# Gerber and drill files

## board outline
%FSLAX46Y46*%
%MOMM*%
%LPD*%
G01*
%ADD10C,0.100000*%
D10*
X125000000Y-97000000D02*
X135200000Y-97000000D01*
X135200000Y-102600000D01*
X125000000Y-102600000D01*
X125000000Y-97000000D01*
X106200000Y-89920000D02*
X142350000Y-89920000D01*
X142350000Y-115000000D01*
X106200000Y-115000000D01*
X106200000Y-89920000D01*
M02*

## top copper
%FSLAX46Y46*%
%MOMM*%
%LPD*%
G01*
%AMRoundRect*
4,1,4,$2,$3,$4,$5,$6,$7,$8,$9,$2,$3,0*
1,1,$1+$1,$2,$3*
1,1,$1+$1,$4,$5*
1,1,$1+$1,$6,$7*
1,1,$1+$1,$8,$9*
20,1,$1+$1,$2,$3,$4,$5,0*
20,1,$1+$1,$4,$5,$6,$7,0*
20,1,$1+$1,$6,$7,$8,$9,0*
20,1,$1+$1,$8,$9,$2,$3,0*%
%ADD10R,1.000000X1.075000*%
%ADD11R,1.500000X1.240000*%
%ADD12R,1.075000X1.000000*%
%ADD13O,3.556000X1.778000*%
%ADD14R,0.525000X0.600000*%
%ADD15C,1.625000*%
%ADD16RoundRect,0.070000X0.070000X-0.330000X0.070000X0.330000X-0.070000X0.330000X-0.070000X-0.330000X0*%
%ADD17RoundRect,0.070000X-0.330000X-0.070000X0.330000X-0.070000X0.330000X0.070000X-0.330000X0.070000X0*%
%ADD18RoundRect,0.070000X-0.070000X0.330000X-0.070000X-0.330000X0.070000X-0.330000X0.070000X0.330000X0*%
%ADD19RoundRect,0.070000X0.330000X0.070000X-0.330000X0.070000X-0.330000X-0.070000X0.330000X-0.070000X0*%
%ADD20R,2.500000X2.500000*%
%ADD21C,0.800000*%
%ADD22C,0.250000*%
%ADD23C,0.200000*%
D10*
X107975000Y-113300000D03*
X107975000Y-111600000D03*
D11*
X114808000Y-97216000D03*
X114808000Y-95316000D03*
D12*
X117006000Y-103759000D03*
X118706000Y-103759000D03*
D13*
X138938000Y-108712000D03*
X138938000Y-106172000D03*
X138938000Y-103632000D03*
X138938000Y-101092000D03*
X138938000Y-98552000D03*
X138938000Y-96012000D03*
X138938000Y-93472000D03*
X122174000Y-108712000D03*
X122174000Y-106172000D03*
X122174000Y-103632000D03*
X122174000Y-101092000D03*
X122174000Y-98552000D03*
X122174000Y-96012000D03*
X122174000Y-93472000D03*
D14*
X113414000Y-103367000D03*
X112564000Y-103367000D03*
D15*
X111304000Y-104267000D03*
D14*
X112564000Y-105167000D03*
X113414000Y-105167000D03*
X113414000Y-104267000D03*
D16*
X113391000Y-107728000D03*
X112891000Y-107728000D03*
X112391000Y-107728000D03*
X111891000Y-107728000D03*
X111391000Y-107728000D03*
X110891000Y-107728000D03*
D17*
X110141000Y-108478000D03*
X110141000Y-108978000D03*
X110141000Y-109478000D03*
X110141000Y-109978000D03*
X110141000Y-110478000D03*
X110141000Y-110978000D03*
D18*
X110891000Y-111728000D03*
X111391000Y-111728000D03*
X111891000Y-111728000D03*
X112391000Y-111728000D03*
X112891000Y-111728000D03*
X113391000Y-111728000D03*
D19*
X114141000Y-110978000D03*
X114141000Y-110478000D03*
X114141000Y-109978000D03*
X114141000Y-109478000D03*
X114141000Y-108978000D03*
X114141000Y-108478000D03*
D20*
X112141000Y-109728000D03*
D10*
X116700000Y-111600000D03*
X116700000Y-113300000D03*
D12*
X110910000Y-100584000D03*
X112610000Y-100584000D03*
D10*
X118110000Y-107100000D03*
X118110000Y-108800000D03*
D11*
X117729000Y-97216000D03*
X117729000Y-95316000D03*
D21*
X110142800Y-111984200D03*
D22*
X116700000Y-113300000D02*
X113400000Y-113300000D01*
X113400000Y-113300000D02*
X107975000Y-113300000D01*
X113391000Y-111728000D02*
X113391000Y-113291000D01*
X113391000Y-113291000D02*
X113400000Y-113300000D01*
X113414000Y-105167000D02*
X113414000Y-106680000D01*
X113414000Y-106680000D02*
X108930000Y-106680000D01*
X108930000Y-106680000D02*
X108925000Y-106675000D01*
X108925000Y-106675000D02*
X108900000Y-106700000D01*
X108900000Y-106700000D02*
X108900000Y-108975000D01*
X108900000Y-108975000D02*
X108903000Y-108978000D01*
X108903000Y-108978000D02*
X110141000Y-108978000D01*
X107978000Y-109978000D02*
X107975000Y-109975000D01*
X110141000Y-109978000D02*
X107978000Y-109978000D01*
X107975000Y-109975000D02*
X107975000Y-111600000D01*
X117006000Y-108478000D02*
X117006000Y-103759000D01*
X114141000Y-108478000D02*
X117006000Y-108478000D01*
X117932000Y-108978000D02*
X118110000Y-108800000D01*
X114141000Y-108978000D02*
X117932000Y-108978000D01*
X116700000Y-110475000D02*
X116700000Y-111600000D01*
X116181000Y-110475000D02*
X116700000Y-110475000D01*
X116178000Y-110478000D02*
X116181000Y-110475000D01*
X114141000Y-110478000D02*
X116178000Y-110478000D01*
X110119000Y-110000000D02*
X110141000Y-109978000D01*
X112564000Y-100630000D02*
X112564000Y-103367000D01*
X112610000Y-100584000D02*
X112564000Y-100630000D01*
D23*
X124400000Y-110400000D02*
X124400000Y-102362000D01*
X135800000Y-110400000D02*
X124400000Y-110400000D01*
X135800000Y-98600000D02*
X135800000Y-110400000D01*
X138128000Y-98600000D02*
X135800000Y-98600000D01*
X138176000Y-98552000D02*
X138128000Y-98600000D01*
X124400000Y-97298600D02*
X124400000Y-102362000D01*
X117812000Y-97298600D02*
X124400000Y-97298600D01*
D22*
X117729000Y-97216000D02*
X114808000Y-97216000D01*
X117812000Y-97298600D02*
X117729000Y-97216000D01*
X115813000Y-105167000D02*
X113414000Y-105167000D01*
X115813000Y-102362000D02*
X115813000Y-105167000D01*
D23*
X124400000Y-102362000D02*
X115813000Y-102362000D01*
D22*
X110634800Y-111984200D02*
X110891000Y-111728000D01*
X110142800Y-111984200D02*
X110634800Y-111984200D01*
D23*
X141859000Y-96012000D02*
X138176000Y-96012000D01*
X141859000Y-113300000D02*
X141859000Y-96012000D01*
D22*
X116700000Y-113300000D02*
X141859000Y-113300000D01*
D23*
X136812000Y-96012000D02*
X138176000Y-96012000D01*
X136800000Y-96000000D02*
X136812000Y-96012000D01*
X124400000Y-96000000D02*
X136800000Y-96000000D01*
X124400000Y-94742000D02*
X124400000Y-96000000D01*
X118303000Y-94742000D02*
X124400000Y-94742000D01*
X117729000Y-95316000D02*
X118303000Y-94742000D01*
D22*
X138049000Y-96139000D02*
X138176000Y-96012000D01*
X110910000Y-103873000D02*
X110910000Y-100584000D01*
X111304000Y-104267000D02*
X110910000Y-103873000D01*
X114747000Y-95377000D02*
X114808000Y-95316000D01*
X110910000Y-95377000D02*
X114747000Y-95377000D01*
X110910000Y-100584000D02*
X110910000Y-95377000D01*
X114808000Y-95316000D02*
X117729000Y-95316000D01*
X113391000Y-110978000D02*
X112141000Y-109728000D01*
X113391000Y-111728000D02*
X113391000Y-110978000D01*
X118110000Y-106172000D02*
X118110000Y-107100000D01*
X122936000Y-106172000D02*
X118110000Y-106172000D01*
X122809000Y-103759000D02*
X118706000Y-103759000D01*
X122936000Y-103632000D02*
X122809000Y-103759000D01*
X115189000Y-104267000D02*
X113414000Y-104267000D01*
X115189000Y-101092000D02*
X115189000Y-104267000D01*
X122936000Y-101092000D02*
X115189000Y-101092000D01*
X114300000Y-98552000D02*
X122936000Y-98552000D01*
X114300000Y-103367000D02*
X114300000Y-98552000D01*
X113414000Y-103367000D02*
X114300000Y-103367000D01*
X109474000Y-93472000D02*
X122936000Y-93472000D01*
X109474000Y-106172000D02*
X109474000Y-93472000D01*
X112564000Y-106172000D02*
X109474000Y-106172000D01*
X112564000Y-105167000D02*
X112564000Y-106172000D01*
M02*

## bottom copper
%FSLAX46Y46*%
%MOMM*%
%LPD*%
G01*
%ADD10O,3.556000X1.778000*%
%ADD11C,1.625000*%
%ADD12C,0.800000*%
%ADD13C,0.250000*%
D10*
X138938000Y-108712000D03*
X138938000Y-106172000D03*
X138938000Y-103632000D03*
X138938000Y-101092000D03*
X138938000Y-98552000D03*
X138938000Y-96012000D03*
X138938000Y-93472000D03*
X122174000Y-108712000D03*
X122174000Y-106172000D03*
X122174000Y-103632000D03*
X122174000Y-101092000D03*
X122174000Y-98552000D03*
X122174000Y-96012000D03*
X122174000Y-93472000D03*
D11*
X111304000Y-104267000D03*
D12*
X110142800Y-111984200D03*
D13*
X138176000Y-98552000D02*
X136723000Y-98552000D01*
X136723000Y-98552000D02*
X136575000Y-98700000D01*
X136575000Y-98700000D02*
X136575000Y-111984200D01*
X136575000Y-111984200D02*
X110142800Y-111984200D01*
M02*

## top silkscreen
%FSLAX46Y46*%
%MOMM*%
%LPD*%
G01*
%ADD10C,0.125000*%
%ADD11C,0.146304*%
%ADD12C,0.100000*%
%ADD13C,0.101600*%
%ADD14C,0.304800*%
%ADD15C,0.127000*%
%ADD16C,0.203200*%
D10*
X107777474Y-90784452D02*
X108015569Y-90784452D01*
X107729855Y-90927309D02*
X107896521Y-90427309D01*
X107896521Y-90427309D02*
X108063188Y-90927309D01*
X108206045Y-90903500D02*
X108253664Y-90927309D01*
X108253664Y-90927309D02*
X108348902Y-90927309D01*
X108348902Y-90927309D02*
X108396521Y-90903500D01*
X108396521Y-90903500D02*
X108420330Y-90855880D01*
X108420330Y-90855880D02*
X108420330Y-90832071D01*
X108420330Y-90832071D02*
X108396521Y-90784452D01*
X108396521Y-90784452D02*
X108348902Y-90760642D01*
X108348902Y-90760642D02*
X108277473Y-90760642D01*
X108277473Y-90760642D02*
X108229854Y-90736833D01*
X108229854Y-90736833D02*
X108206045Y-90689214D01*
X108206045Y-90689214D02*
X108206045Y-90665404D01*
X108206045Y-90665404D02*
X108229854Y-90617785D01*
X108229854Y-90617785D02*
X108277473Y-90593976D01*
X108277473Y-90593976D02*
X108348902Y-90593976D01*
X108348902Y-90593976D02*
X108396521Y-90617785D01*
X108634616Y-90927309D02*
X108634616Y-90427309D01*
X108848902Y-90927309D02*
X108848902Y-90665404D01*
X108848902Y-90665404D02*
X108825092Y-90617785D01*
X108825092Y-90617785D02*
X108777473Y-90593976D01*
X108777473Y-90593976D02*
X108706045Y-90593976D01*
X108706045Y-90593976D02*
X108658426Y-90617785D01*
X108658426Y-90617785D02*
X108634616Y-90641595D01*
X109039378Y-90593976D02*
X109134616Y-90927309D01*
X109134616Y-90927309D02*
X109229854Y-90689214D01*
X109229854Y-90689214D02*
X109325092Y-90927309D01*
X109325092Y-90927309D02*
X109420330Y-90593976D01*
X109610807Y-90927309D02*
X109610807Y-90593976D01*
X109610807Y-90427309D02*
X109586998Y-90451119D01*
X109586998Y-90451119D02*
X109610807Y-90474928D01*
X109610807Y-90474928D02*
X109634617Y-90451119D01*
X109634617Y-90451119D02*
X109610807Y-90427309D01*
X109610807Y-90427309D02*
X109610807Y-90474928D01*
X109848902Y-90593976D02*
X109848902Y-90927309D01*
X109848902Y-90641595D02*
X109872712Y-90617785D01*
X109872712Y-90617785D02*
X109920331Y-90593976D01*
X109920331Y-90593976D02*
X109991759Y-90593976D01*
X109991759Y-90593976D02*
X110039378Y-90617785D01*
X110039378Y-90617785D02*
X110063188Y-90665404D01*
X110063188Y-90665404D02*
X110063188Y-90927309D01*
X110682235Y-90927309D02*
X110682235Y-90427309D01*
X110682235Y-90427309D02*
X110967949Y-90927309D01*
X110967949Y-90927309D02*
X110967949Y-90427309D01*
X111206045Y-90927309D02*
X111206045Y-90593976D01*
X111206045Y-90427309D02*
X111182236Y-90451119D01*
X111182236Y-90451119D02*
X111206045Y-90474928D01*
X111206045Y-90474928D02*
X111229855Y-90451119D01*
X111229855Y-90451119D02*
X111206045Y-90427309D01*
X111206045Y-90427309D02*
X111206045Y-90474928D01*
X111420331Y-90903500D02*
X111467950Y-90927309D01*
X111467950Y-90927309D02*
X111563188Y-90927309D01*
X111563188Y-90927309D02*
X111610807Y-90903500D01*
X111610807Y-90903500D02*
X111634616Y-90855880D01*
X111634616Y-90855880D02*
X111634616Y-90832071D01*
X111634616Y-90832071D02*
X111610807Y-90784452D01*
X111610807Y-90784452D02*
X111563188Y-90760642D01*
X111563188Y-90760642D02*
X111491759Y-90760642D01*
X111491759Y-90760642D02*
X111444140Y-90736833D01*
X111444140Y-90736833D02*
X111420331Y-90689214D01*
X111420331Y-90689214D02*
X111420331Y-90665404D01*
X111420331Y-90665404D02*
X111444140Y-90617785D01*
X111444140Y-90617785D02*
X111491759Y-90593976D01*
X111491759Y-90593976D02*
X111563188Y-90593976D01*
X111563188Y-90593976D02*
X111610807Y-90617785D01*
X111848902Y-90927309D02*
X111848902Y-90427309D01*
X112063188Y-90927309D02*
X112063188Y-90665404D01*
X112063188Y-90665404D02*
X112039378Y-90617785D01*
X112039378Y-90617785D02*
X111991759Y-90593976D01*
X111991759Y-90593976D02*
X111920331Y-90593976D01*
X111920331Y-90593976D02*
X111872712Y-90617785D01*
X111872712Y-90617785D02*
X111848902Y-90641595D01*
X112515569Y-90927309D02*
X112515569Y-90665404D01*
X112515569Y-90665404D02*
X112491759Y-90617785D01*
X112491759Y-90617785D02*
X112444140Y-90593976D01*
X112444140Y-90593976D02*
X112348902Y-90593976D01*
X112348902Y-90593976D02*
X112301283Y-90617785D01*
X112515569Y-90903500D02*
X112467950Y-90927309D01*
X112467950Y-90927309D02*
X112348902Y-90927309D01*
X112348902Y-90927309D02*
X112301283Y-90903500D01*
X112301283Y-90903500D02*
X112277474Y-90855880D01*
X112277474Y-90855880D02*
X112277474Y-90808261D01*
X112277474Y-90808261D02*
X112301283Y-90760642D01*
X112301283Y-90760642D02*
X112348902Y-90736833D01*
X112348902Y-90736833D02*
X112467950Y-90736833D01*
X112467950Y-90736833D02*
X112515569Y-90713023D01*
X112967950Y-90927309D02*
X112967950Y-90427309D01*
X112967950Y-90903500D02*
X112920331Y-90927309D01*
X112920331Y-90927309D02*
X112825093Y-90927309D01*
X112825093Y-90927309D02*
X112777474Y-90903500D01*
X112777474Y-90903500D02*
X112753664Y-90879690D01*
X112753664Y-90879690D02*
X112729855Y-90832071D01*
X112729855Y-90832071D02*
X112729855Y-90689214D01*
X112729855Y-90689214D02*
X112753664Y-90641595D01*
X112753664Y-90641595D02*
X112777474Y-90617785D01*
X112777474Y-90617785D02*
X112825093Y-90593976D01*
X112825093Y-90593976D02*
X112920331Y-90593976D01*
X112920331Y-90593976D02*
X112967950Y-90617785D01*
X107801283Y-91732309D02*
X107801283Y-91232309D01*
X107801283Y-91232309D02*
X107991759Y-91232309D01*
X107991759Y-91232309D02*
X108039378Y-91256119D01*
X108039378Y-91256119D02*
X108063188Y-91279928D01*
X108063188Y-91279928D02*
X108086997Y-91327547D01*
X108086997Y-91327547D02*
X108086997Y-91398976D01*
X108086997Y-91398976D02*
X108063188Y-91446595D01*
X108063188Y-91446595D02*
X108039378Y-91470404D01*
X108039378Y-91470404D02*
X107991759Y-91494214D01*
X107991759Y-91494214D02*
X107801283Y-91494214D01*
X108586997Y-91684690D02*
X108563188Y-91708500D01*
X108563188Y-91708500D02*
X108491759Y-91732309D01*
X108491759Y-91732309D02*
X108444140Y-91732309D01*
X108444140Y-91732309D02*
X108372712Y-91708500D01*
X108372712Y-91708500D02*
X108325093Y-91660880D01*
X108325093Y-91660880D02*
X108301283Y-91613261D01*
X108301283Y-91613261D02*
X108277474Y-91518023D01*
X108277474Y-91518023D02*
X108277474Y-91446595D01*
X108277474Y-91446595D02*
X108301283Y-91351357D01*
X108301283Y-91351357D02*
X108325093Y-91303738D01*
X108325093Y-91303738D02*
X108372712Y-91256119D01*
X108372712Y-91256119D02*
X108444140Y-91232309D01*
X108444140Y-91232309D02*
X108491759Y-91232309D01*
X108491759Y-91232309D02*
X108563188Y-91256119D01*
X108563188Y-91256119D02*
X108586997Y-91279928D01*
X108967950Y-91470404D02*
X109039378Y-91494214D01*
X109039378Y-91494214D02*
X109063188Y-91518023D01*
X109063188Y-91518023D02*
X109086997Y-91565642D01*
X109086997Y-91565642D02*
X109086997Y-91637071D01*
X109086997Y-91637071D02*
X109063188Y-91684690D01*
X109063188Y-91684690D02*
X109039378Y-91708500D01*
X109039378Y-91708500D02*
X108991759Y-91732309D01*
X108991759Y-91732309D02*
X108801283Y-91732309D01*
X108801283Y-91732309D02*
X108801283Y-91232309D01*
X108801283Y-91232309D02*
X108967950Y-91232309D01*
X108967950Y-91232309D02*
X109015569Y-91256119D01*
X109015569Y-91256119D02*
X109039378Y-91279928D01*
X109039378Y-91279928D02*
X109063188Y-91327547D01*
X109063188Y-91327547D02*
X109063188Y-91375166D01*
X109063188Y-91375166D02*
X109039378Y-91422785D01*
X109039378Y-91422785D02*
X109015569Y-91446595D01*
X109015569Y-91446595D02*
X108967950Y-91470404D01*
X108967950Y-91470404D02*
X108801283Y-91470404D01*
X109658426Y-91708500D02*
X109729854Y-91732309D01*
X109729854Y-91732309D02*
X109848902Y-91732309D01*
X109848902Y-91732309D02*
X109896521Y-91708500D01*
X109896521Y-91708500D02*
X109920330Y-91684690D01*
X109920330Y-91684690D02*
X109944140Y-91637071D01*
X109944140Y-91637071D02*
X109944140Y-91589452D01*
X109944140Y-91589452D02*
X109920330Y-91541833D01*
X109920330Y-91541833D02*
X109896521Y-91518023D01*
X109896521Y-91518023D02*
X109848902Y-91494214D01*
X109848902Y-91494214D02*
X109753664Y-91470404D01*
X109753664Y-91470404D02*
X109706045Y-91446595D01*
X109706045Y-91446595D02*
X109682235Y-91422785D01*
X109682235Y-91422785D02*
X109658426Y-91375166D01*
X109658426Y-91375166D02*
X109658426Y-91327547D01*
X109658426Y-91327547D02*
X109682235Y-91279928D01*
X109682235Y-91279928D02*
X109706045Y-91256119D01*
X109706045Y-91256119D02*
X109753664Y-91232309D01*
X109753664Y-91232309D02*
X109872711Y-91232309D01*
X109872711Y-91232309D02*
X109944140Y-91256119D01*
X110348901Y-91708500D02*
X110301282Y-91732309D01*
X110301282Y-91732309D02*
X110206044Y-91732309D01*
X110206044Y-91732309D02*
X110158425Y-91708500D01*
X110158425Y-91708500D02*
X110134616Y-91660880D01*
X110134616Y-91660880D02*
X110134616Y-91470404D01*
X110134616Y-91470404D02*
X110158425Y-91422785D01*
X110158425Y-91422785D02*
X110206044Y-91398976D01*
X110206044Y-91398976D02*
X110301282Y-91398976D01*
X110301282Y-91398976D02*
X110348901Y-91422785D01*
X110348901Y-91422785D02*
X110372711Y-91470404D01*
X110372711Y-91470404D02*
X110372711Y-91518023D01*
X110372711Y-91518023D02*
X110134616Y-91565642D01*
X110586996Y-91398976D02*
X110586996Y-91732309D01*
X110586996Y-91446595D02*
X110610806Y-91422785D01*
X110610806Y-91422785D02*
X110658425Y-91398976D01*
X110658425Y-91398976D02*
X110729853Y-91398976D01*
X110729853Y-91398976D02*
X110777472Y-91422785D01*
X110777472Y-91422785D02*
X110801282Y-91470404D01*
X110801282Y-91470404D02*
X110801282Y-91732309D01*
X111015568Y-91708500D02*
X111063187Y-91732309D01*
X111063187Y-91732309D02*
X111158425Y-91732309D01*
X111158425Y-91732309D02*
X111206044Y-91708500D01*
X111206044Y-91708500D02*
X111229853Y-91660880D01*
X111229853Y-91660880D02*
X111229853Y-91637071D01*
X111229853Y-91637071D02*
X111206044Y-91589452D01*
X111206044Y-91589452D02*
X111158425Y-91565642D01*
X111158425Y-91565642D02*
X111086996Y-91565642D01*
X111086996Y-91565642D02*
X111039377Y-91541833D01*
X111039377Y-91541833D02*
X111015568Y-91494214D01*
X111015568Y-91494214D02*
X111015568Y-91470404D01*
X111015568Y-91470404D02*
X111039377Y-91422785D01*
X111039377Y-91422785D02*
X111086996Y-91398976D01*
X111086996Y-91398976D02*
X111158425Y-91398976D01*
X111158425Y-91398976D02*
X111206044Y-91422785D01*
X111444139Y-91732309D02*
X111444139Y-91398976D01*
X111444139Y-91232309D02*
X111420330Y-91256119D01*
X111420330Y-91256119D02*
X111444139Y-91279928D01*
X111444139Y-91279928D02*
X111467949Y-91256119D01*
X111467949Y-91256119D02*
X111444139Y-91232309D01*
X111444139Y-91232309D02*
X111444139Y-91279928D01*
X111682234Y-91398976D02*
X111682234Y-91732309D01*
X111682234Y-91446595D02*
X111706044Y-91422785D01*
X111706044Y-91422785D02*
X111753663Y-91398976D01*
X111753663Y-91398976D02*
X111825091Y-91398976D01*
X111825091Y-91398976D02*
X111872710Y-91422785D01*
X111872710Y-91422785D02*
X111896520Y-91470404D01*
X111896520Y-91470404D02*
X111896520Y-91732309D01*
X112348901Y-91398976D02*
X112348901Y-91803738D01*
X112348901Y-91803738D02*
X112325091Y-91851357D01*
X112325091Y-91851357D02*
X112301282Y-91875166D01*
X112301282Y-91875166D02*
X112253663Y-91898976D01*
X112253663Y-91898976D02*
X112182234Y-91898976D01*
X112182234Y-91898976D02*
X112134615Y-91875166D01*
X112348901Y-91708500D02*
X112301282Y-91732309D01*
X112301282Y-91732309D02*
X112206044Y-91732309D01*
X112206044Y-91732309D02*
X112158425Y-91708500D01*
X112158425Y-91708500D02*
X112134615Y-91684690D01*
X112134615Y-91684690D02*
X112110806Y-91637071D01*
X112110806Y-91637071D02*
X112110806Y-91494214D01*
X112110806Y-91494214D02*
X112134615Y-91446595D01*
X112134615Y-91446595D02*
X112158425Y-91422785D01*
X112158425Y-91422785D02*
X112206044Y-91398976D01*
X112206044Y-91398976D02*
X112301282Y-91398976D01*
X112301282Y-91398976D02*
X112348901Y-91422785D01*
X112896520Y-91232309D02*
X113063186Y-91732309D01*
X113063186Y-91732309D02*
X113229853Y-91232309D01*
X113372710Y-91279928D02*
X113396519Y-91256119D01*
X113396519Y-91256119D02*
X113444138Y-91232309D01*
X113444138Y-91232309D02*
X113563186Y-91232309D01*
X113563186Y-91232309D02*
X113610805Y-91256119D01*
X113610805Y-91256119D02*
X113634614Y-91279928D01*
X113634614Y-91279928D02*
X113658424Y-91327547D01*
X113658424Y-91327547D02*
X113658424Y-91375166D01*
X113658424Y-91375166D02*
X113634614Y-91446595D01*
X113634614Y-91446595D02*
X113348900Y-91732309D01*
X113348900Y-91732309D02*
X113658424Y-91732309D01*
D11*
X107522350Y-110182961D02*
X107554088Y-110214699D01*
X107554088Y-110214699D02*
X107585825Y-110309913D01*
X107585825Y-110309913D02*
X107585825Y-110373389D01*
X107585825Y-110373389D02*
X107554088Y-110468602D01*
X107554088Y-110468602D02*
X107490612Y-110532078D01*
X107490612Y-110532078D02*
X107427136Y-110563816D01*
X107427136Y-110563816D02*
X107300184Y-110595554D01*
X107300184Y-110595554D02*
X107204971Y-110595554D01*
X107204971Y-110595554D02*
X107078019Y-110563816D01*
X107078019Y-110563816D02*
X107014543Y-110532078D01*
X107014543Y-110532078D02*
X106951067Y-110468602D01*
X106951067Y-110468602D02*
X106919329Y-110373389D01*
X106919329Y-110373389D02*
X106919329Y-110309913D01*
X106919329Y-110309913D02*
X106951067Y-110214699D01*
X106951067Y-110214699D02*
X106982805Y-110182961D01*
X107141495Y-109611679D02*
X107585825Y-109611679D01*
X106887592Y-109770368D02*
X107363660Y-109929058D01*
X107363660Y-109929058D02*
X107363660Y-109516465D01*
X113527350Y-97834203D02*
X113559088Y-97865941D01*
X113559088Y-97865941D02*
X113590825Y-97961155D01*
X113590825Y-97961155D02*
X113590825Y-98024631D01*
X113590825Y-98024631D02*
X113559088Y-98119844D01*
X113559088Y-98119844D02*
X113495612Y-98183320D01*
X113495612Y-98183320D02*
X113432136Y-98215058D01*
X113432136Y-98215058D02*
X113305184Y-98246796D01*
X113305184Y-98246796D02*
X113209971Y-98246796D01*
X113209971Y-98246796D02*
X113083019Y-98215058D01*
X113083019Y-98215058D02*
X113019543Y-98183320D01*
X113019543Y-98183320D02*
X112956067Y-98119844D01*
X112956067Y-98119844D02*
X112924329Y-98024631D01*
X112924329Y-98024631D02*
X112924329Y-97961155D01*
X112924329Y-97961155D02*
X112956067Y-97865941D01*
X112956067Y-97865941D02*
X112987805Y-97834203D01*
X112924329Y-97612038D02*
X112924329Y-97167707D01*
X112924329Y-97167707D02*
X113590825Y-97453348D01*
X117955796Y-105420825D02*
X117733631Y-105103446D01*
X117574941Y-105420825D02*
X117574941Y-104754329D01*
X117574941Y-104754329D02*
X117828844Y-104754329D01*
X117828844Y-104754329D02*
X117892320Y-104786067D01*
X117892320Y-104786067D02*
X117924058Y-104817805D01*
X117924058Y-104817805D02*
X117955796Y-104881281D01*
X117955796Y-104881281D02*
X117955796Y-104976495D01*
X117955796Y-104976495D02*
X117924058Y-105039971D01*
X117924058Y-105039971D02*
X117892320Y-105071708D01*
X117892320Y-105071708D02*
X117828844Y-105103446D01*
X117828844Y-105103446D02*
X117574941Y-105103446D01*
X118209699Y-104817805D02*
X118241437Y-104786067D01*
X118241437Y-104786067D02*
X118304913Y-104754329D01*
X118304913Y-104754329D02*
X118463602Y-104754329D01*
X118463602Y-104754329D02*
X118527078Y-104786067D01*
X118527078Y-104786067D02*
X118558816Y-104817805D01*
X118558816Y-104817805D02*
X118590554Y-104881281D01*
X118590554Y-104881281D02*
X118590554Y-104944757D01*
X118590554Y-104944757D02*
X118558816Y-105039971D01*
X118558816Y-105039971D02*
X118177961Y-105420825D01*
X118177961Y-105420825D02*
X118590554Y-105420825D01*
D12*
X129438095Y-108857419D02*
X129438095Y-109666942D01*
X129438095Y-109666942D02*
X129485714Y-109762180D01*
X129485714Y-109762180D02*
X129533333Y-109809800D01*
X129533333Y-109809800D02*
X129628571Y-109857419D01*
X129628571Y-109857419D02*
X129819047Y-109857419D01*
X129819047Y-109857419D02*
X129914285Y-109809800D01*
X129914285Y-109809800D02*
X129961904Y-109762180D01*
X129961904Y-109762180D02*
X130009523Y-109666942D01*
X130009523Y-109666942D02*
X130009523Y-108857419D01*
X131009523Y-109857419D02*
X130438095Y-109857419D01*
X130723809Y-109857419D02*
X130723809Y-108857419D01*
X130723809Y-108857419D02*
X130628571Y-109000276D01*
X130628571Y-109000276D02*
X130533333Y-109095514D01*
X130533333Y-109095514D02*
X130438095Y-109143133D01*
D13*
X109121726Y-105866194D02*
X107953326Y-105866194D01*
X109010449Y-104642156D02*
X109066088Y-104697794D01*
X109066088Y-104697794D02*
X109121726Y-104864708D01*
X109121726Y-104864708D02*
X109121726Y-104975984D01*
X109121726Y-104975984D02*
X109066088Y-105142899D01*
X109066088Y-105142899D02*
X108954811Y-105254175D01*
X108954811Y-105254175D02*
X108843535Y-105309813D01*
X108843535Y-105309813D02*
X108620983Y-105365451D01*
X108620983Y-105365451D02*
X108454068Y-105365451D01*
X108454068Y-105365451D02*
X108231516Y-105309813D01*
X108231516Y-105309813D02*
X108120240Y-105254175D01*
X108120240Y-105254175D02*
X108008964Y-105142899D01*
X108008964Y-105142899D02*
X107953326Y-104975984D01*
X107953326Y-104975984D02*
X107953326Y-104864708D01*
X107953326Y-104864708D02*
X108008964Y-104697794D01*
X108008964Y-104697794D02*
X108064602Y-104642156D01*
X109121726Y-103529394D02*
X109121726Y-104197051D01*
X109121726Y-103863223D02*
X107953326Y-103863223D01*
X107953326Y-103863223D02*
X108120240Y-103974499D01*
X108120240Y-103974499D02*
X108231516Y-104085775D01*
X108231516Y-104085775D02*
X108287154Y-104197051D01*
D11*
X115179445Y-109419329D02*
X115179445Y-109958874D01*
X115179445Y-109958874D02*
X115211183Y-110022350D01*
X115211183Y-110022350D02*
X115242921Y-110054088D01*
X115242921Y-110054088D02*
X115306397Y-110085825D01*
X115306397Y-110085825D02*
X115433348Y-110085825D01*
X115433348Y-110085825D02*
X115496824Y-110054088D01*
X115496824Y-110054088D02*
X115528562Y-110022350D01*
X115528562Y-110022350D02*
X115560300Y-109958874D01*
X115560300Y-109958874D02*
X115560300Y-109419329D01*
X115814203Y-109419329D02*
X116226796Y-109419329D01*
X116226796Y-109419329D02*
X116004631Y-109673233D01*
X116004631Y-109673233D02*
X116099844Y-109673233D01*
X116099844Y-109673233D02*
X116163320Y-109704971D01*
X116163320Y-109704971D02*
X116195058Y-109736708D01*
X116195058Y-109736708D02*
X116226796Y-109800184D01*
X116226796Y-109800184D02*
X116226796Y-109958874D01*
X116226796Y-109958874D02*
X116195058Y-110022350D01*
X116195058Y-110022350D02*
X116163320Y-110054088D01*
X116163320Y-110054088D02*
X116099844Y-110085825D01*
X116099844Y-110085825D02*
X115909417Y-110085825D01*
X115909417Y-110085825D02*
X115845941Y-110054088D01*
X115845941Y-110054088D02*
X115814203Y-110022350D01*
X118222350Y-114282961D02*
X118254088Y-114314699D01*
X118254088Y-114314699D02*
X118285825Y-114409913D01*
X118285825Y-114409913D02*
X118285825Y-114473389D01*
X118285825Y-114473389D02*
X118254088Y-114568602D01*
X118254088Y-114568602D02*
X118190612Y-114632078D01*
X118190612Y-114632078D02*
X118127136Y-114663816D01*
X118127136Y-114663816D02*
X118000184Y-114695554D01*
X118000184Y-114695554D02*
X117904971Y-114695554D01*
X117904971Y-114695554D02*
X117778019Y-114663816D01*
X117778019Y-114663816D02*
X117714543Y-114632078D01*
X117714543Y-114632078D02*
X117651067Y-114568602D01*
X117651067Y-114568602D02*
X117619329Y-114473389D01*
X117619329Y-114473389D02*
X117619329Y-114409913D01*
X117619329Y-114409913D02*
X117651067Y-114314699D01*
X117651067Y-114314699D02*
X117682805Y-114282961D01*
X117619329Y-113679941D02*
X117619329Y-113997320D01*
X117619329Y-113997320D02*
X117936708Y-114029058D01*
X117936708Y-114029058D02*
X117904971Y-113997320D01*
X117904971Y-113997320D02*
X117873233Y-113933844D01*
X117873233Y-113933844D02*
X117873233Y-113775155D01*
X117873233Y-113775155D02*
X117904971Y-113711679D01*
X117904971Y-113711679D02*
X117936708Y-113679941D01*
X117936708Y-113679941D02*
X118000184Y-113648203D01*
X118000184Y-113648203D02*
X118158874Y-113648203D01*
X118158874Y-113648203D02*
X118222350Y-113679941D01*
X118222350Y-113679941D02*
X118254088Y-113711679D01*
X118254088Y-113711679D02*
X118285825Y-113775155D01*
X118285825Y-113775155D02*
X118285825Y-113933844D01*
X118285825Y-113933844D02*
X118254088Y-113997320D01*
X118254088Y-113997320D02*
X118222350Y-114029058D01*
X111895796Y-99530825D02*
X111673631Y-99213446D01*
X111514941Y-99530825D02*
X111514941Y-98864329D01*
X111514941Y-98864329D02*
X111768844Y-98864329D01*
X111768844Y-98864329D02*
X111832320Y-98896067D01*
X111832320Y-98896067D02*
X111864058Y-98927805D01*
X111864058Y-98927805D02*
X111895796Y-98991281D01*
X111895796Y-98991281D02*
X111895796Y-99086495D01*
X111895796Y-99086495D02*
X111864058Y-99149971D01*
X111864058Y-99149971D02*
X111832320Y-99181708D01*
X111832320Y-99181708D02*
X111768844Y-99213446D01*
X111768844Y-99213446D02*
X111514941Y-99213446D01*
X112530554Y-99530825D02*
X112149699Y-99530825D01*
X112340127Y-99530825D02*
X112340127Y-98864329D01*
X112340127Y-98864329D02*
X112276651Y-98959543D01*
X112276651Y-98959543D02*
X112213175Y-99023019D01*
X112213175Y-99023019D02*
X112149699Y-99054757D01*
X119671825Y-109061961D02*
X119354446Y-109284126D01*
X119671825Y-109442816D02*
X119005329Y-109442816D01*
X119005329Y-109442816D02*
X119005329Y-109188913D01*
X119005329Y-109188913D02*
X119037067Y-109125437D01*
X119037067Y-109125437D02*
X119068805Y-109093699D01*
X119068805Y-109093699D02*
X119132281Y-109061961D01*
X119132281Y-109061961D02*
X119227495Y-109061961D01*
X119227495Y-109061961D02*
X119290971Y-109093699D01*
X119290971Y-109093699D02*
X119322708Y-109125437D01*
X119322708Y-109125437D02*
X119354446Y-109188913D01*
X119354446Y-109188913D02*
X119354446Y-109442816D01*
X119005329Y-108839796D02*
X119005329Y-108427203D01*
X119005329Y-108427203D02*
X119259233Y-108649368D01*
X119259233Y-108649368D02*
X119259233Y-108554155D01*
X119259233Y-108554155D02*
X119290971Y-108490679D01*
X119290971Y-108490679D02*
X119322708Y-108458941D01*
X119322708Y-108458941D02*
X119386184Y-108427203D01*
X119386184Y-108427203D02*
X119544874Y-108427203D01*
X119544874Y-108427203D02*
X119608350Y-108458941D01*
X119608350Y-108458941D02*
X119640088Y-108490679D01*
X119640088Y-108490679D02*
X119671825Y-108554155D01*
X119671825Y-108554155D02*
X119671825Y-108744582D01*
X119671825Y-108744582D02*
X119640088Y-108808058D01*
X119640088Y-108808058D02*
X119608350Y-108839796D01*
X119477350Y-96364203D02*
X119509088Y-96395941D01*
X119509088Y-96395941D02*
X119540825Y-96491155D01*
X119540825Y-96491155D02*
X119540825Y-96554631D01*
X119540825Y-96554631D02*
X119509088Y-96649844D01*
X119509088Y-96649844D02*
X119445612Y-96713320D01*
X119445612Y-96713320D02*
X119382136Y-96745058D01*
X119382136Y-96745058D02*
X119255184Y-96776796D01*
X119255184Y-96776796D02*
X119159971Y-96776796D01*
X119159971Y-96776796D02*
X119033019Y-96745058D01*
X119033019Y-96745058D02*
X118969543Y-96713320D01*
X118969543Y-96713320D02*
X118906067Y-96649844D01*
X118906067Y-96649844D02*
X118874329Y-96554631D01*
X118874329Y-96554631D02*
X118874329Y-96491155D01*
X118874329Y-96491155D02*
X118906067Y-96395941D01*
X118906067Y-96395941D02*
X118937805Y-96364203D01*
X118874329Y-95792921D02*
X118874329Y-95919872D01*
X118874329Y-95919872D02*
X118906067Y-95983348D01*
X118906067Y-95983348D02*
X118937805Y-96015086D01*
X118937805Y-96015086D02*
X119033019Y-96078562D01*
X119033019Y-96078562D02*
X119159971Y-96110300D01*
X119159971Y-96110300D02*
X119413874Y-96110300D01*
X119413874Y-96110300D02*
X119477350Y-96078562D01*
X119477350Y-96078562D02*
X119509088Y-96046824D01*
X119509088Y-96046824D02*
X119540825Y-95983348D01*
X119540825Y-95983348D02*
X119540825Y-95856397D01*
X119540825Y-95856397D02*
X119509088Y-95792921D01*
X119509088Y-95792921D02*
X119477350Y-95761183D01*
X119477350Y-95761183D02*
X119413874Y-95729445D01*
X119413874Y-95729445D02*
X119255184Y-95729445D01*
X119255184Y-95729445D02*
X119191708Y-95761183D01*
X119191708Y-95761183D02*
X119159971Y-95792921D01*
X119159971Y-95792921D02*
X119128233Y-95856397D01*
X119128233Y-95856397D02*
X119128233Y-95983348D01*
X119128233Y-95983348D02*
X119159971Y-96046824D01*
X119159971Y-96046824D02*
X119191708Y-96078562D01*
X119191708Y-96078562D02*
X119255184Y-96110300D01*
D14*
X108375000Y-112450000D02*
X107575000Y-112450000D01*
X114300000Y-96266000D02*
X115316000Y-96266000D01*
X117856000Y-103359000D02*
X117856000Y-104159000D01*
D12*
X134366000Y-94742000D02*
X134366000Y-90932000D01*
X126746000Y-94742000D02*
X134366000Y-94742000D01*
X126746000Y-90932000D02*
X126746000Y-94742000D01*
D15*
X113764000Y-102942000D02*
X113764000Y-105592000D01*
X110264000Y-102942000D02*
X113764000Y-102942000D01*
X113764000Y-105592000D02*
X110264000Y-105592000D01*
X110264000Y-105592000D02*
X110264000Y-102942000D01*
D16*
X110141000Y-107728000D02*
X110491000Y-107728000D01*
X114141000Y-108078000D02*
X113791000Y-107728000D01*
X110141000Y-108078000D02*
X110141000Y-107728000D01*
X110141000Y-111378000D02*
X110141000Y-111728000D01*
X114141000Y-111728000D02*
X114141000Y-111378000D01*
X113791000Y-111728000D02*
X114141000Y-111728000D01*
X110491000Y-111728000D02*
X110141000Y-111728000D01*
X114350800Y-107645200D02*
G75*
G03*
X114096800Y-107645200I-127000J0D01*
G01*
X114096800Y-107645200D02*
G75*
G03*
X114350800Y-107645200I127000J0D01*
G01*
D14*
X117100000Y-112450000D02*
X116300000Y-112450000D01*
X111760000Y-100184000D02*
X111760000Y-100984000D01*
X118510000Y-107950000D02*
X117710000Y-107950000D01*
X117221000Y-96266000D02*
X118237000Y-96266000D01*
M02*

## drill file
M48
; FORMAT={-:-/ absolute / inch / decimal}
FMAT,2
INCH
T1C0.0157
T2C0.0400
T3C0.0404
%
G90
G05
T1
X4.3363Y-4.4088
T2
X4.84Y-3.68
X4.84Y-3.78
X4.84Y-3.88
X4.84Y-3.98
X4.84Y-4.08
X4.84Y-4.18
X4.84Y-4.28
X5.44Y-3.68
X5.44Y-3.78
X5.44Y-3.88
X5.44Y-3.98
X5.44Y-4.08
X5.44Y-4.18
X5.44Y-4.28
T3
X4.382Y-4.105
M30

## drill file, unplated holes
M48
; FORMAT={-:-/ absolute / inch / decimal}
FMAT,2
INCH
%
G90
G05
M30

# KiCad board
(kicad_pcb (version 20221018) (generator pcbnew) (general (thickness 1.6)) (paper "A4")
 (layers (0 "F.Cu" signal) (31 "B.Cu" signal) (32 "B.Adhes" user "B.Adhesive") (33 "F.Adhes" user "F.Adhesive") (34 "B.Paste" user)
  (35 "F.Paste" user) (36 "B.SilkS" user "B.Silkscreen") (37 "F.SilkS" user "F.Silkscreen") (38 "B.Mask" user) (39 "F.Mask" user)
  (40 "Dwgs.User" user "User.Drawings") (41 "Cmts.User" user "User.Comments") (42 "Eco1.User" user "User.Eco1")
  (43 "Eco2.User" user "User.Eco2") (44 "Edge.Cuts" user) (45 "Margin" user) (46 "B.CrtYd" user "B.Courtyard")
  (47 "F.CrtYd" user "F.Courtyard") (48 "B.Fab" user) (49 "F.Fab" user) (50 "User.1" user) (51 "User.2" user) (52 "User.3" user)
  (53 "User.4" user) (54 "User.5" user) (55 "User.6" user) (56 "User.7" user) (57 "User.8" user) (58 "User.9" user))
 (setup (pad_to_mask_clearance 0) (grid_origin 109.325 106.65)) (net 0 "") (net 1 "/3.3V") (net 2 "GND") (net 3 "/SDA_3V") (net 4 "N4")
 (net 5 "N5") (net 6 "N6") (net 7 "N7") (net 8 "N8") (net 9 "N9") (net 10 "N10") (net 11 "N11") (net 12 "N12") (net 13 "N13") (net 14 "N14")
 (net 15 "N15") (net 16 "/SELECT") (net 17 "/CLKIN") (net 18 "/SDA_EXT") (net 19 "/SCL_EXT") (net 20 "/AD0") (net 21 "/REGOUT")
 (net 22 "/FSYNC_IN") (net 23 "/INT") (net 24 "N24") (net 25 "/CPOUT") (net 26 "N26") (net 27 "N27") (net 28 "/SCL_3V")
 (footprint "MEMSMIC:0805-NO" (layer "F.Cu") (at 114.808 96.266 90)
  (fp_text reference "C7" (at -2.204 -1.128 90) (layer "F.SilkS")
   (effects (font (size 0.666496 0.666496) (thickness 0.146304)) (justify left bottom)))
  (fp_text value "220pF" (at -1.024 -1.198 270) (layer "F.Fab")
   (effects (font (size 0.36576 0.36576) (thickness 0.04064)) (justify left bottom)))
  (fp_line (start 0 -0.508) (end 0 0.508) (stroke (width 0.3048) (type solid)) (layer "F.SilkS"))
  (pad "1" smd rect (at -0.95 0 90) (size 1.24 1.5) (layers "F.Cu" "F.Paste" "F.Mask") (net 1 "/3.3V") (solder_mask_margin 0.0508)
   (thermal_bridge_angle 0))
  (pad "2" smd rect (at 0.95 0 90) (size 1.24 1.5) (layers "F.Cu" "F.Paste" "F.Mask") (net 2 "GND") (solder_mask_margin 0.0508)
   (thermal_bridge_angle 0)))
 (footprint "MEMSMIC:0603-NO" (layer "F.Cu") (at 117.856 103.759)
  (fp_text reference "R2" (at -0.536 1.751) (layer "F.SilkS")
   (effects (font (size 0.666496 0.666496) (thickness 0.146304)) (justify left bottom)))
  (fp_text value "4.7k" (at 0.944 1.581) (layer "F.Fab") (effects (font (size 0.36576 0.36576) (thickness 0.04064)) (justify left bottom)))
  (fp_line (start 0 -0.4) (end 0 0.4) (stroke (width 0.3048) (type solid)) (layer "F.SilkS"))
  (pad "1" smd rect (at -0.85 0) (size 1.075 1) (layers "F.Cu" "F.Paste" "F.Mask") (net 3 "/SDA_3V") (solder_mask_margin 0.0508)
   (thermal_bridge_angle 0))
  (pad "2" smd rect (at 0.85 0) (size 1.075 1) (layers "F.Cu" "F.Paste" "F.Mask") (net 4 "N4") (solder_mask_margin 0.0508)
   (thermal_bridge_angle 0)))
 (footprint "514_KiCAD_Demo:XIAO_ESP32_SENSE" (layer "F.Cu") (at 130.556 101.092)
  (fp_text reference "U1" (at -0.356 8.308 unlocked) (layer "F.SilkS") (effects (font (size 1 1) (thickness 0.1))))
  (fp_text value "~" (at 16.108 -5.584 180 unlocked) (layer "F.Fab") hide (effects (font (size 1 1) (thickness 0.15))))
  (fp_line (start -3.81 -10.16) (end -3.81 -6.35) (stroke (width 0.1) (type default)) (layer "F.SilkS"))
  (fp_line (start -3.81 -6.35) (end 3.81 -6.35) (stroke (width 0.1) (type default)) (layer "F.SilkS"))
  (fp_line (start 3.81 -6.35) (end 3.81 -10.16) (stroke (width 0.1) (type default)) (layer "F.SilkS"))
  (pad "1" thru_hole oval (at -7.62 -7.62) (size 3.556 1.778) (drill 1.016 (offset -0.762 0)) (layers "*.Cu" "*.Mask") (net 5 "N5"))
  (pad "2" thru_hole oval (at -7.62 -5.08) (size 3.556 1.778) (drill 1.016 (offset -0.762 0)) (layers "*.Cu" "*.Mask") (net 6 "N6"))
  (pad "3" thru_hole oval (at -7.62 -2.54) (size 3.556 1.778) (drill 1.016 (offset -0.762 0)) (layers "*.Cu" "*.Mask") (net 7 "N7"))
  (pad "4" thru_hole oval (at -7.62 0) (size 3.556 1.778) (drill 1.016 (offset -0.762 0)) (layers "*.Cu" "*.Mask") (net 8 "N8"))
  (pad "5" thru_hole oval (at -7.62 2.54) (size 3.556 1.778) (drill 1.016 (offset -0.762 0)) (layers "*.Cu" "*.Mask") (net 4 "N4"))
  (pad "6" thru_hole oval (at -7.62 5.08) (size 3.556 1.778) (drill 1.016 (offset -0.762 0)) (layers "*.Cu" "*.Mask") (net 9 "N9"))
  (pad "7" thru_hole oval (at -7.62 7.62) (size 3.556 1.778) (drill 1.016 (offset -0.762 0)) (layers "*.Cu" "*.Mask") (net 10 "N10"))
  (pad "8" thru_hole oval (at 7.62 -7.62) (size 3.556 1.778) (drill 1.016 (offset 0.762 0)) (layers "*.Cu" "*.Mask") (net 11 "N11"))
  (pad "9" thru_hole oval (at 7.62 -5.08) (size 3.556 1.778) (drill 1.016 (offset 0.762 0)) (layers "*.Cu" "*.Mask") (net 2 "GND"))
  (pad "10" thru_hole oval (at 7.62 -2.54) (size 3.556 1.778) (drill 1.016 (offset 0.762 0)) (layers "*.Cu" "*.Mask") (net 1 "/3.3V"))
  (pad "11" thru_hole oval (at 7.62 0) (size 3.556 1.778) (drill 1.016 (offset 0.762 0)) (layers "*.Cu" "*.Mask") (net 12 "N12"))
  (pad "12" thru_hole oval (at 7.62 2.54) (size 3.556 1.778) (drill 1.016 (offset 0.762 0)) (layers "*.Cu" "*.Mask") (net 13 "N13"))
  (pad "13" thru_hole oval (at 7.62 5.08) (size 3.556 1.778) (drill 1.016 (offset 0.762 0)) (layers "*.Cu" "*.Mask") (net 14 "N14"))
  (pad "14" thru_hole oval (at 7.62 7.62) (size 3.556 1.778) (drill 1.016 (offset 0.762 0)) (layers "*.Cu" "*.Mask") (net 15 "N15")))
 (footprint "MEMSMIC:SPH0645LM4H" (layer "F.Cu") (at 112.014 104.267 -90)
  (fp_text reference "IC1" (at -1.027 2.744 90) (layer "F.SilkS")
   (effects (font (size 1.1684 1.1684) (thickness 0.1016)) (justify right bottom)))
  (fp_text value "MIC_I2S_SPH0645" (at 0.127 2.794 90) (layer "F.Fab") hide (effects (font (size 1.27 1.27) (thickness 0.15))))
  (fp_line (start -1.325 -1.75) (end 1.325 -1.75) (stroke (width 0.127) (type solid)) (layer "F.SilkS"))
  (fp_line (start -1.325 1.75) (end -1.325 -1.75) (stroke (width 0.127) (type solid)) (layer "F.SilkS"))
  (fp_line (start 1.325 -1.75) (end 1.325 1.75) (stroke (width 0.127) (type solid)) (layer "F.SilkS"))
  (fp_line (start 1.325 1.75) (end -1.325 1.75) (stroke (width 0.127) (type solid)) (layer "F.SilkS"))
  (pad "1" smd rect (at -0.9 -1.4 270) (size 0.6 0.525) (layers "F.Cu" "F.Paste" "F.Mask") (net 7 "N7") (solder_mask_margin 0.0508)
   (thermal_bridge_angle 0))
  (pad "2" smd rect (at -0.9 -0.55 270) (size 0.6 0.525) (layers "F.Cu" "F.Paste" "F.Mask") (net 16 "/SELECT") (solder_mask_margin 0.0508)
   (thermal_bridge_angle 0))
  (pad "3" thru_hole circle (at 0 0.71 270) (size 1.625 1.625) (drill 1.025) (layers "*.Cu" "*.Mask") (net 2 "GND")
   (solder_mask_margin 0.0508) (thermal_bridge_angle 0))
  (pad "4" smd rect (at 0.9 -0.55 270) (size 0.6 0.525) (layers "F.Cu" "F.Paste" "F.Mask") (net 5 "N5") (solder_mask_margin 0.0508)
   (thermal_bridge_angle 0))
  (pad "5" smd rect (at 0.9 -1.4 270) (size 0.6 0.525) (layers "F.Cu" "F.Paste" "F.Mask") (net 1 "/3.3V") (solder_mask_margin 0.0508)
   (thermal_bridge_angle 0))
  (pad "6" smd rect (at 0 -1.4 270) (size 0.6 0.525) (layers "F.Cu" "F.Paste" "F.Mask") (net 8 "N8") (solder_mask_margin 0.0508)
   (thermal_bridge_angle 0)))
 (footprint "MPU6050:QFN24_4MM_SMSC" (layer "F.Cu") (at 112.141 109.728 -90)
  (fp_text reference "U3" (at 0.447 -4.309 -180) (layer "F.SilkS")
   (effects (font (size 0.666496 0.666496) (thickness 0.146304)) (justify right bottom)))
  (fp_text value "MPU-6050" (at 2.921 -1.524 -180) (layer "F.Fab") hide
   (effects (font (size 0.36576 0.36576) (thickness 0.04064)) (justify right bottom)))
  (fp_line (start -2 2) (end -2 1.65) (stroke (width 0.2032) (type solid)) (layer "F.SilkS"))
  (fp_line (start -1.65 -2) (end -2 -1.65) (stroke (width 0.2032) (type solid)) (layer "F.SilkS"))
  (fp_line (start -1.65 2) (end -2 2) (stroke (width 0.2032) (type solid)) (layer "F.SilkS"))
  (fp_line (start 1.65 2) (end 2 2) (stroke (width 0.2032) (type solid)) (layer "F.SilkS"))
  (fp_line (start 2 -2) (end 1.65 -2) (stroke (width 0.2032) (type solid)) (layer "F.SilkS"))
  (fp_line (start 2 -1.65) (end 2 -2) (stroke (width 0.2032) (type solid)) (layer "F.SilkS"))
  (fp_line (start 2 1.65) (end 2 2) (stroke (width 0.2032) (type solid)) (layer "F.SilkS"))
  (fp_circle (center -2.0828 -2.0828) (end -1.9558 -2.0828) (stroke (width 0.2032) (type solid)) (fill none) (layer "F.SilkS"))
  (pad "1" smd roundrect (at -2 -1.25 90) (size 0.8 0.28) (layers "F.Cu" "F.Paste" "F.Mask") (roundrect_rratio 0.25) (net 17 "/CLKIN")
   (solder_mask_margin 0.0508) (thermal_bridge_angle 0))
  (pad "2" smd roundrect (at -2 -0.75 90) (size 0.8 0.28) (layers "F.Cu" "F.Paste" "F.Mask") (roundrect_rratio 0.25)
   (solder_mask_margin 0.0508) (thermal_bridge_angle 0))
  (pad "3" smd roundrect (at -2 -0.25 90) (size 0.8 0.28) (layers "F.Cu" "F.Paste" "F.Mask") (roundrect_rratio 0.25)
   (solder_mask_margin 0.0508) (thermal_bridge_angle 0))
  (pad "4" smd roundrect (at -2 0.25 90) (size 0.8 0.28) (layers "F.Cu" "F.Paste" "F.Mask") (roundrect_rratio 0.25)
   (solder_mask_margin 0.0508) (thermal_bridge_angle 0))
  (pad "5" smd roundrect (at -2 0.75 90) (size 0.8 0.28) (layers "F.Cu" "F.Paste" "F.Mask") (roundrect_rratio 0.25)
   (solder_mask_margin 0.0508) (thermal_bridge_angle 0))
  (pad "6" smd roundrect (at -2 1.25 90) (size 0.8 0.28) (layers "F.Cu" "F.Paste" "F.Mask") (roundrect_rratio 0.25) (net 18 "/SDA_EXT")
   (solder_mask_margin 0.0508) (thermal_bridge_angle 0))
  (pad "7" smd roundrect (at -1.25 2) (size 0.8 0.28) (layers "F.Cu" "F.Paste" "F.Mask") (roundrect_rratio 0.25) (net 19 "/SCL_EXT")
   (solder_mask_margin 0.0508) (thermal_bridge_angle 0))
  (pad "8" smd roundrect (at -0.75 2) (size 0.8 0.28) (layers "F.Cu" "F.Paste" "F.Mask") (roundrect_rratio 0.25) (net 1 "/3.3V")
   (solder_mask_margin 0.0508) (thermal_bridge_angle 0))
  (pad "9" smd roundrect (at -0.25 2) (size 0.8 0.28) (layers "F.Cu" "F.Paste" "F.Mask") (roundrect_rratio 0.25) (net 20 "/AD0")
   (solder_mask_margin 0.0508) (thermal_bridge_angle 0))
  (pad "10" smd roundrect (at 0.25 2) (size 0.8 0.28) (layers "F.Cu" "F.Paste" "F.Mask") (roundrect_rratio 0.25) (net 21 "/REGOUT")
   (solder_mask_margin 0.0508) (thermal_bridge_angle 0))
  (pad "11" smd roundrect (at 0.75 2) (size 0.8 0.28) (layers "F.Cu" "F.Paste" "F.Mask") (roundrect_rratio 0.25) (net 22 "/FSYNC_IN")
   (solder_mask_margin 0.0508) (thermal_bridge_angle 0))
  (pad "12" smd roundrect (at 1.25 2) (size 0.8 0.28) (layers "F.Cu" "F.Paste" "F.Mask") (roundrect_rratio 0.25) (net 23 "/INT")
   (solder_mask_margin 0.0508) (thermal_bridge_angle 0))
  (pad "13" smd roundrect (at 2 1.25 270) (size 0.8 0.28) (layers "F.Cu" "F.Paste" "F.Mask") (roundrect_rratio 0.25) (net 1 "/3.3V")
   (solder_mask_margin 0.0508) (thermal_bridge_angle 0))
  (pad "14" smd roundrect (at 2 0.75 270) (size 0.8 0.28) (layers "F.Cu" "F.Paste" "F.Mask") (roundrect_rratio 0.25)
   (solder_mask_margin 0.0508) (thermal_bridge_angle 0))
  (pad "15" smd roundrect (at 2 0.25 270) (size 0.8 0.28) (layers "F.Cu" "F.Paste" "F.Mask") (roundrect_rratio 0.25)
   (solder_mask_margin 0.0508) (thermal_bridge_angle 0))
  (pad "16" smd roundrect (at 2 -0.25 270) (size 0.8 0.28) (layers "F.Cu" "F.Paste" "F.Mask") (roundrect_rratio 0.25)
   (solder_mask_margin 0.0508) (thermal_bridge_angle 0))
  (pad "17" smd roundrect (at 2 -0.75 270) (size 0.8 0.28) (layers "F.Cu" "F.Paste" "F.Mask") (roundrect_rratio 0.25)
   (solder_mask_margin 0.0508) (thermal_bridge_angle 0))
  (pad "18" smd roundrect (at 2 -1.25 270) (size 0.8 0.28) (layers "F.Cu" "F.Paste" "F.Mask") (roundrect_rratio 0.25) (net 2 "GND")
   (solder_mask_margin 0.0508) (thermal_bridge_angle 0))
  (pad "19" smd roundrect (at 1.25 -2 180) (size 0.8 0.28) (layers "F.Cu" "F.Paste" "F.Mask") (roundrect_rratio 0.25) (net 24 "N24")
   (solder_mask_margin 0.0508) (thermal_bridge_angle 0))
  (pad "20" smd roundrect (at 0.75 -2 180) (size 0.8 0.28) (layers "F.Cu" "F.Paste" "F.Mask") (roundrect_rratio 0.25) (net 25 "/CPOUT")
   (solder_mask_margin 0.0508) (thermal_bridge_angle 0))
  (pad "21" smd roundrect (at 0.25 -2 180) (size 0.8 0.28) (layers "F.Cu" "F.Paste" "F.Mask") (roundrect_rratio 0.25) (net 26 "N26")
   (solder_mask_margin 0.0508) (thermal_bridge_angle 0))
  (pad "22" smd roundrect (at -0.25 -2 180) (size 0.8 0.28) (layers "F.Cu" "F.Paste" "F.Mask") (roundrect_rratio 0.25) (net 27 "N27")
   (solder_mask_margin 0.0508) (thermal_bridge_angle 0))
  (pad "23" smd roundrect (at -0.75 -2 180) (size 0.8 0.28) (layers "F.Cu" "F.Paste" "F.Mask") (roundrect_rratio 0.25) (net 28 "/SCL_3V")
   (solder_mask_margin 0.0508) (thermal_bridge_angle 0))
  (pad "24" smd roundrect (at -1.25 -2 180) (size 0.8 0.28) (layers "F.Cu" "F.Paste" "F.Mask") (roundrect_rratio 0.25) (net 3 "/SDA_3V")
   (solder_mask_margin 0.0508) (thermal_bridge_angle 0))
  (pad "THERM" smd rect (at 0 0 270) (size 2.5 2.5) (layers "F.Cu" "F.Mask") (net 2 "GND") (solder_mask_margin 0.0508)
   (thermal_bridge_angle 0)))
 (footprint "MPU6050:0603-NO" (layer "F.Cu") (at 116.7 112.45 -90)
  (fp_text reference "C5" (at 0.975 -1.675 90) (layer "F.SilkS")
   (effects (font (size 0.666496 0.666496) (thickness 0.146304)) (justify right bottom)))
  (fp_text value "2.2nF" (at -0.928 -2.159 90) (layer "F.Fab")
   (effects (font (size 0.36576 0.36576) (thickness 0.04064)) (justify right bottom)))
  (fp_line (start 0 -0.4) (end 0 0.4) (stroke (width 0.3048) (type solid)) (layer "F.SilkS"))
  (pad "1" smd rect (at -0.85 0 270) (size 1.075 1) (layers "F.Cu" "F.Paste" "F.Mask") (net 25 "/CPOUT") (solder_mask_margin 0.0508)
   (thermal_bridge_angle 0))
  (pad "2" smd rect (at 0.85 0 270) (size 1.075 1) (layers "F.Cu" "F.Paste" "F.Mask") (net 2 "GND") (solder_mask_margin 0.0508)
   (thermal_bridge_angle 0)))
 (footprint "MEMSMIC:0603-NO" (layer "F.Cu") (at 111.76 100.584)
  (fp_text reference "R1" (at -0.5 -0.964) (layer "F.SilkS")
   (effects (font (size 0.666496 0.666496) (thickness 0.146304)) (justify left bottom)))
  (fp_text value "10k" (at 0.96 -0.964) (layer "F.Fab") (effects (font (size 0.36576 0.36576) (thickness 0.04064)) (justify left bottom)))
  (fp_line (start 0 -0.4) (end 0 0.4) (stroke (width 0.3048) (type solid)) (layer "F.SilkS"))
  (pad "1" smd rect (at -0.85 0) (size 1.075 1) (layers "F.Cu" "F.Paste" "F.Mask") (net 2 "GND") (solder_mask_margin 0.0508)
   (thermal_bridge_angle 0))
  (pad "2" smd rect (at 0.85 0) (size 1.075 1) (layers "F.Cu" "F.Paste" "F.Mask") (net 16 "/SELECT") (solder_mask_margin 0.0508)
   (thermal_bridge_angle 0)))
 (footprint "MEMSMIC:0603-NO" (layer "F.Cu") (at 118.11 107.95 -90)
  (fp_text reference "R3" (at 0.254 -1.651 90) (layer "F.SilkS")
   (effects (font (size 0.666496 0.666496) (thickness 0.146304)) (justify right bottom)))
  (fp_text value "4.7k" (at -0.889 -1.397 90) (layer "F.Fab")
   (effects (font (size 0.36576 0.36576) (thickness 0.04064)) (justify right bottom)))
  (fp_line (start 0 -0.4) (end 0 0.4) (stroke (width 0.3048) (type solid)) (layer "F.SilkS"))
  (pad "1" smd rect (at -0.85 0 270) (size 1.075 1) (layers "F.Cu" "F.Paste" "F.Mask") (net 9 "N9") (solder_mask_margin 0.0508)
   (thermal_bridge_angle 0))
  (pad "2" smd rect (at 0.85 0 270) (size 1.075 1) (layers "F.Cu" "F.Paste" "F.Mask") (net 28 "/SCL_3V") (solder_mask_margin 0.0508)
   (thermal_bridge_angle 0)))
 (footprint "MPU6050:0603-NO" (layer "F.Cu") (at 107.975 112.45 -90)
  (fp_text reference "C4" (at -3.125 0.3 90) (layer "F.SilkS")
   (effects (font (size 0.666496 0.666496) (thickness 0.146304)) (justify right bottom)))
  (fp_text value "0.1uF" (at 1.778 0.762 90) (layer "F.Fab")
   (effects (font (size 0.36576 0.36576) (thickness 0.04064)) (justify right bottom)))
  (fp_line (start 0 -0.4) (end 0 0.4) (stroke (width 0.3048) (type solid)) (layer "F.SilkS"))
  (pad "1" smd rect (at -0.85 0 270) (size 1.075 1) (layers "F.Cu" "F.Paste" "F.Mask") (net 21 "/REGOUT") (solder_mask_margin 0.0508)
   (thermal_bridge_angle 0))
  (pad "2" smd rect (at 0.85 0 270) (size 1.075 1) (layers "F.Cu" "F.Paste" "F.Mask") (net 2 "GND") (solder_mask_margin 0.0508)
   (thermal_bridge_angle 0)))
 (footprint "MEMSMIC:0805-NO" (layer "F.Cu") (at 117.729 96.266 90)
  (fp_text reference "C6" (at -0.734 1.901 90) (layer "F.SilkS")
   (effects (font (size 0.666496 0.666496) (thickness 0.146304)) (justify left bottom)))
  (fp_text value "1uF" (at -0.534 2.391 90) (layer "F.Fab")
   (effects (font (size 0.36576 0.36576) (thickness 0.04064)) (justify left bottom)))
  (fp_line (start 0 -0.508) (end 0 0.508) (stroke (width 0.3048) (type solid)) (layer "F.SilkS"))
  (pad "1" smd rect (at -0.95 0 90) (size 1.24 1.5) (layers "F.Cu" "F.Paste" "F.Mask") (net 1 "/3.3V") (solder_mask_margin 0.0508)
   (thermal_bridge_angle 0))
  (pad "2" smd rect (at 0.95 0 90) (size 1.24 1.5) (layers "F.Cu" "F.Paste" "F.Mask") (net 2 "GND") (solder_mask_margin 0.0508)
   (thermal_bridge_angle 0)))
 (gr_rect (start 125 97) (end 135.2 102.6) (stroke (width 0.1) (type default)) (fill none) (layer "Edge.Cuts"))
 (gr_rect (start 106.2 89.92) (end 142.35 115) (stroke (width 0.1) (type default)) (fill none) (layer "Edge.Cuts"))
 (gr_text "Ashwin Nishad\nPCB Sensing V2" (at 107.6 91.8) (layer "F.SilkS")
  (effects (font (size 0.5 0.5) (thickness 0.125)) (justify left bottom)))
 (segment (start 112.564 105.167) (end 112.564 106.172) (width 0.25) (layer "F.Cu") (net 5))
 (segment (start 109.474 106.172) (end 109.474 93.472) (width 0.25) (layer "F.Cu") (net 5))
 (segment (start 109.474 93.472) (end 122.936 93.472) (width 0.25) (layer "F.Cu") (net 5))
 (segment (start 112.564 106.172) (end 109.474 106.172) (width 0.25) (layer "F.Cu") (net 5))
 (segment (start 113.414 103.367) (end 114.3 103.367) (width 0.25) (layer "F.Cu") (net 7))
 (segment (start 114.3 103.367) (end 114.3 98.552) (width 0.25) (layer "F.Cu") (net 7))
 (segment (start 114.3 98.552) (end 122.936 98.552) (width 0.25) (layer "F.Cu") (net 7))
 (segment (start 115.189 101.092) (end 115.189 104.267) (width 0.25) (layer "F.Cu") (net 8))
 (segment (start 115.189 104.267) (end 113.414 104.267) (width 0.25) (layer "F.Cu") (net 8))
 (segment (start 122.936 101.092) (end 115.189 101.092) (width 0.25) (layer "F.Cu") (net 8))
 (segment (start 122.936 103.632) (end 122.809 103.759) (width 0.25) (layer "F.Cu") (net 4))
 (segment (start 122.809 103.759) (end 118.706 103.759) (width 0.25) (layer "F.Cu") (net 4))
 (segment (start 122.936 106.172) (end 118.11 106.172) (width 0.25) (layer "F.Cu") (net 9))
 (segment (start 118.11 106.172) (end 118.11 107.1) (width 0.25) (layer "F.Cu") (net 9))
 (segment (start 138.049 96.139) (end 138.176 96.012) (width 0.25) (layer "F.Cu") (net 2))
 (segment (start 136.8 96) (end 136.812 96.012) (width 0.2) (layer "F.Cu") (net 2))
 (segment (start 118.303 94.742) (end 124.4 94.742) (width 0.2) (layer "F.Cu") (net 2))
 (segment (start 110.91 95.377) (end 114.747 95.377) (width 0.25) (layer "F.Cu") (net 2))
 (segment (start 113.391 111.728) (end 113.391 113.291) (width 0.25) (layer "F.Cu") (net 2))
 (segment (start 113.391 110.978) (end 112.141 109.728) (width 0.25) (layer "F.Cu") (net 2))
 (segment (start 124.4 96) (end 136.8 96) (width 0.2) (layer "F.Cu") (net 2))
 (segment (start 110.91 103.873) (end 110.91 100.584) (width 0.25) (layer "F.Cu") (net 2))
 (segment (start 136.812 96.012) (end 138.176 96.012) (width 0.2) (layer "F.Cu") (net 2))
 (segment (start 110.91 100.584) (end 110.91 95.377) (width 0.25) (layer "F.Cu") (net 2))
 (segment (start 117.729 95.316) (end 118.303 94.742) (width 0.2) (layer "F.Cu") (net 2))
 (segment (start 116.7 113.3) (end 141.859 113.3) (width 0.25) (layer "F.Cu") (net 2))
 (segment (start 113.4 113.3) (end 107.975 113.3) (width 0.25) (layer "F.Cu") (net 2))
 (segment (start 114.747 95.377) (end 114.808 95.316) (width 0.25) (layer "F.Cu") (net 2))
 (segment (start 141.859 113.3) (end 141.859 96.012) (width 0.2) (layer "F.Cu") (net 2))
 (segment (start 114.808 95.316) (end 117.729 95.316) (width 0.25) (layer "F.Cu") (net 2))
 (segment (start 113.391 113.291) (end 113.4 113.3) (width 0.25) (layer "F.Cu") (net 2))
 (segment (start 116.7 113.3) (end 113.4 113.3) (width 0.25) (layer "F.Cu") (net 2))
 (segment (start 113.391 111.728) (end 113.391 110.978) (width 0.25) (layer "F.Cu") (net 2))
 (segment (start 111.304 104.267) (end 110.91 103.873) (width 0.25) (layer "F.Cu") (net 2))
 (segment (start 124.4 94.742) (end 124.4 96) (width 0.2) (layer "F.Cu") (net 2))
 (segment (start 141.859 96.012) (end 138.176 96.012) (width 0.2) (layer "F.Cu") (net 2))
 (segment (start 115.813 102.362) (end 115.813 105.167) (width 0.25) (layer "F.Cu") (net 1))
 (segment (start 110.1428 111.9842) (end 110.6348 111.9842) (width 0.25) (layer "F.Cu") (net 1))
 (segment (start 135.8 110.4) (end 124.4 110.4) (width 0.2) (layer "F.Cu") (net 1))
 (segment (start 113.414 106.68) (end 108.93 106.68) (width 0.25) (layer "F.Cu") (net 1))
 (segment (start 108.925 106.675) (end 108.9 106.7) (width 0.25) (layer "F.Cu") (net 1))
 (segment (start 108.93 106.68) (end 108.925 106.675) (width 0.25) (layer "F.Cu") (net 1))
 (segment (start 138.128 98.6) (end 135.8 98.6) (width 0.2) (layer "F.Cu") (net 1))
 (segment (start 117.729 97.216) (end 114.808 97.216) (width 0.25) (layer "F.Cu") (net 1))
 (segment (start 124.4 102.362) (end 115.813 102.362) (width 0.2) (layer "F.Cu") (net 1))
 (segment (start 110.6348 111.9842) (end 110.891 111.728) (width 0.25) (layer "F.Cu") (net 1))
 (segment (start 117.812 97.2986) (end 117.729 97.216) (width 0.25) (layer "F.Cu") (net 1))
 (segment (start 108.9 106.7) (end 108.9 108.975) (width 0.25) (layer "F.Cu") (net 1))
 (segment (start 135.8 98.6) (end 135.8 110.4) (width 0.2) (layer "F.Cu") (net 1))
 (segment (start 117.812 97.2986) (end 124.4 97.2986) (width 0.2) (layer "F.Cu") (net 1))
 (segment (start 138.176 98.552) (end 138.128 98.6) (width 0.2) (layer "F.Cu") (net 1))
 (segment (start 108.9 108.975) (end 108.903 108.978) (width 0.25) (layer "F.Cu") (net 1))
 (segment (start 124.4 110.4) (end 124.4 102.362) (width 0.2) (layer "F.Cu") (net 1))
 (segment (start 108.903 108.978) (end 110.141 108.978) (width 0.25) (layer "F.Cu") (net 1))
 (segment (start 124.4 97.2986) (end 124.4 102.362) (width 0.2) (layer "F.Cu") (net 1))
 (segment (start 113.414 105.167) (end 113.414 106.68) (width 0.25) (layer "F.Cu") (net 1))
 (segment (start 115.813 105.167) (end 113.414 105.167) (width 0.25) (layer "F.Cu") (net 1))
 (via (at 110.1428 111.9842) (size 0.8) (drill 0.4) (layers "F.Cu" "B.Cu") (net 1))
 (segment (start 136.575 111.9842) (end 110.1428 111.9842) (width 0.25) (layer "B.Cu") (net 1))
 (segment (start 138.176 98.552) (end 136.723 98.552) (width 0.25) (layer "B.Cu") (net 1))
 (segment (start 136.723 98.552) (end 136.575 98.7) (width 0.25) (layer "B.Cu") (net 1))
 (segment (start 136.575 98.7) (end 136.575 111.9842) (width 0.25) (layer "B.Cu") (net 1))
 (segment (start 112.564 100.63) (end 112.564 103.367) (width 0.25) (layer "F.Cu") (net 16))
 (segment (start 112.61 100.584) (end 112.564 100.63) (width 0.25) (layer "F.Cu") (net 16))
 (segment (start 107.975 109.975) (end 107.975 111.6) (width 0.25) (layer "F.Cu") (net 21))
 (segment (start 110.119 110) (end 110.141 109.978) (width 0.25) (layer "F.Cu") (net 21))
 (segment (start 110.141 109.978) (end 107.978 109.978) (width 0.25) (layer "F.Cu") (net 21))
 (segment (start 107.978 109.978) (end 107.975 109.975) (width 0.25) (layer "F.Cu") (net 21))
 (segment (start 116.7 110.475) (end 116.7 111.6) (width 0.25) (layer "F.Cu") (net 25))
 (segment (start 116.178 110.478) (end 116.181 110.475) (width 0.25) (layer "F.Cu") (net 25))
 (segment (start 116.181 110.475) (end 116.7 110.475) (width 0.25) (layer "F.Cu") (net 25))
 (segment (start 114.141 110.478) (end 116.178 110.478) (width 0.25) (layer "F.Cu") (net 25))
 (segment (start 114.141 108.978) (end 117.932 108.978) (width 0.25) (layer "F.Cu") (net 28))
 (segment (start 117.932 108.978) (end 118.11 108.8) (width 0.25) (layer "F.Cu") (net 28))
 (segment (start 114.141 108.478) (end 117.006 108.478) (width 0.25) (layer "F.Cu") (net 3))
 (segment (start 117.006 108.478) (end 117.006 103.759) (width 0.25) (layer "F.Cu") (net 3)))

